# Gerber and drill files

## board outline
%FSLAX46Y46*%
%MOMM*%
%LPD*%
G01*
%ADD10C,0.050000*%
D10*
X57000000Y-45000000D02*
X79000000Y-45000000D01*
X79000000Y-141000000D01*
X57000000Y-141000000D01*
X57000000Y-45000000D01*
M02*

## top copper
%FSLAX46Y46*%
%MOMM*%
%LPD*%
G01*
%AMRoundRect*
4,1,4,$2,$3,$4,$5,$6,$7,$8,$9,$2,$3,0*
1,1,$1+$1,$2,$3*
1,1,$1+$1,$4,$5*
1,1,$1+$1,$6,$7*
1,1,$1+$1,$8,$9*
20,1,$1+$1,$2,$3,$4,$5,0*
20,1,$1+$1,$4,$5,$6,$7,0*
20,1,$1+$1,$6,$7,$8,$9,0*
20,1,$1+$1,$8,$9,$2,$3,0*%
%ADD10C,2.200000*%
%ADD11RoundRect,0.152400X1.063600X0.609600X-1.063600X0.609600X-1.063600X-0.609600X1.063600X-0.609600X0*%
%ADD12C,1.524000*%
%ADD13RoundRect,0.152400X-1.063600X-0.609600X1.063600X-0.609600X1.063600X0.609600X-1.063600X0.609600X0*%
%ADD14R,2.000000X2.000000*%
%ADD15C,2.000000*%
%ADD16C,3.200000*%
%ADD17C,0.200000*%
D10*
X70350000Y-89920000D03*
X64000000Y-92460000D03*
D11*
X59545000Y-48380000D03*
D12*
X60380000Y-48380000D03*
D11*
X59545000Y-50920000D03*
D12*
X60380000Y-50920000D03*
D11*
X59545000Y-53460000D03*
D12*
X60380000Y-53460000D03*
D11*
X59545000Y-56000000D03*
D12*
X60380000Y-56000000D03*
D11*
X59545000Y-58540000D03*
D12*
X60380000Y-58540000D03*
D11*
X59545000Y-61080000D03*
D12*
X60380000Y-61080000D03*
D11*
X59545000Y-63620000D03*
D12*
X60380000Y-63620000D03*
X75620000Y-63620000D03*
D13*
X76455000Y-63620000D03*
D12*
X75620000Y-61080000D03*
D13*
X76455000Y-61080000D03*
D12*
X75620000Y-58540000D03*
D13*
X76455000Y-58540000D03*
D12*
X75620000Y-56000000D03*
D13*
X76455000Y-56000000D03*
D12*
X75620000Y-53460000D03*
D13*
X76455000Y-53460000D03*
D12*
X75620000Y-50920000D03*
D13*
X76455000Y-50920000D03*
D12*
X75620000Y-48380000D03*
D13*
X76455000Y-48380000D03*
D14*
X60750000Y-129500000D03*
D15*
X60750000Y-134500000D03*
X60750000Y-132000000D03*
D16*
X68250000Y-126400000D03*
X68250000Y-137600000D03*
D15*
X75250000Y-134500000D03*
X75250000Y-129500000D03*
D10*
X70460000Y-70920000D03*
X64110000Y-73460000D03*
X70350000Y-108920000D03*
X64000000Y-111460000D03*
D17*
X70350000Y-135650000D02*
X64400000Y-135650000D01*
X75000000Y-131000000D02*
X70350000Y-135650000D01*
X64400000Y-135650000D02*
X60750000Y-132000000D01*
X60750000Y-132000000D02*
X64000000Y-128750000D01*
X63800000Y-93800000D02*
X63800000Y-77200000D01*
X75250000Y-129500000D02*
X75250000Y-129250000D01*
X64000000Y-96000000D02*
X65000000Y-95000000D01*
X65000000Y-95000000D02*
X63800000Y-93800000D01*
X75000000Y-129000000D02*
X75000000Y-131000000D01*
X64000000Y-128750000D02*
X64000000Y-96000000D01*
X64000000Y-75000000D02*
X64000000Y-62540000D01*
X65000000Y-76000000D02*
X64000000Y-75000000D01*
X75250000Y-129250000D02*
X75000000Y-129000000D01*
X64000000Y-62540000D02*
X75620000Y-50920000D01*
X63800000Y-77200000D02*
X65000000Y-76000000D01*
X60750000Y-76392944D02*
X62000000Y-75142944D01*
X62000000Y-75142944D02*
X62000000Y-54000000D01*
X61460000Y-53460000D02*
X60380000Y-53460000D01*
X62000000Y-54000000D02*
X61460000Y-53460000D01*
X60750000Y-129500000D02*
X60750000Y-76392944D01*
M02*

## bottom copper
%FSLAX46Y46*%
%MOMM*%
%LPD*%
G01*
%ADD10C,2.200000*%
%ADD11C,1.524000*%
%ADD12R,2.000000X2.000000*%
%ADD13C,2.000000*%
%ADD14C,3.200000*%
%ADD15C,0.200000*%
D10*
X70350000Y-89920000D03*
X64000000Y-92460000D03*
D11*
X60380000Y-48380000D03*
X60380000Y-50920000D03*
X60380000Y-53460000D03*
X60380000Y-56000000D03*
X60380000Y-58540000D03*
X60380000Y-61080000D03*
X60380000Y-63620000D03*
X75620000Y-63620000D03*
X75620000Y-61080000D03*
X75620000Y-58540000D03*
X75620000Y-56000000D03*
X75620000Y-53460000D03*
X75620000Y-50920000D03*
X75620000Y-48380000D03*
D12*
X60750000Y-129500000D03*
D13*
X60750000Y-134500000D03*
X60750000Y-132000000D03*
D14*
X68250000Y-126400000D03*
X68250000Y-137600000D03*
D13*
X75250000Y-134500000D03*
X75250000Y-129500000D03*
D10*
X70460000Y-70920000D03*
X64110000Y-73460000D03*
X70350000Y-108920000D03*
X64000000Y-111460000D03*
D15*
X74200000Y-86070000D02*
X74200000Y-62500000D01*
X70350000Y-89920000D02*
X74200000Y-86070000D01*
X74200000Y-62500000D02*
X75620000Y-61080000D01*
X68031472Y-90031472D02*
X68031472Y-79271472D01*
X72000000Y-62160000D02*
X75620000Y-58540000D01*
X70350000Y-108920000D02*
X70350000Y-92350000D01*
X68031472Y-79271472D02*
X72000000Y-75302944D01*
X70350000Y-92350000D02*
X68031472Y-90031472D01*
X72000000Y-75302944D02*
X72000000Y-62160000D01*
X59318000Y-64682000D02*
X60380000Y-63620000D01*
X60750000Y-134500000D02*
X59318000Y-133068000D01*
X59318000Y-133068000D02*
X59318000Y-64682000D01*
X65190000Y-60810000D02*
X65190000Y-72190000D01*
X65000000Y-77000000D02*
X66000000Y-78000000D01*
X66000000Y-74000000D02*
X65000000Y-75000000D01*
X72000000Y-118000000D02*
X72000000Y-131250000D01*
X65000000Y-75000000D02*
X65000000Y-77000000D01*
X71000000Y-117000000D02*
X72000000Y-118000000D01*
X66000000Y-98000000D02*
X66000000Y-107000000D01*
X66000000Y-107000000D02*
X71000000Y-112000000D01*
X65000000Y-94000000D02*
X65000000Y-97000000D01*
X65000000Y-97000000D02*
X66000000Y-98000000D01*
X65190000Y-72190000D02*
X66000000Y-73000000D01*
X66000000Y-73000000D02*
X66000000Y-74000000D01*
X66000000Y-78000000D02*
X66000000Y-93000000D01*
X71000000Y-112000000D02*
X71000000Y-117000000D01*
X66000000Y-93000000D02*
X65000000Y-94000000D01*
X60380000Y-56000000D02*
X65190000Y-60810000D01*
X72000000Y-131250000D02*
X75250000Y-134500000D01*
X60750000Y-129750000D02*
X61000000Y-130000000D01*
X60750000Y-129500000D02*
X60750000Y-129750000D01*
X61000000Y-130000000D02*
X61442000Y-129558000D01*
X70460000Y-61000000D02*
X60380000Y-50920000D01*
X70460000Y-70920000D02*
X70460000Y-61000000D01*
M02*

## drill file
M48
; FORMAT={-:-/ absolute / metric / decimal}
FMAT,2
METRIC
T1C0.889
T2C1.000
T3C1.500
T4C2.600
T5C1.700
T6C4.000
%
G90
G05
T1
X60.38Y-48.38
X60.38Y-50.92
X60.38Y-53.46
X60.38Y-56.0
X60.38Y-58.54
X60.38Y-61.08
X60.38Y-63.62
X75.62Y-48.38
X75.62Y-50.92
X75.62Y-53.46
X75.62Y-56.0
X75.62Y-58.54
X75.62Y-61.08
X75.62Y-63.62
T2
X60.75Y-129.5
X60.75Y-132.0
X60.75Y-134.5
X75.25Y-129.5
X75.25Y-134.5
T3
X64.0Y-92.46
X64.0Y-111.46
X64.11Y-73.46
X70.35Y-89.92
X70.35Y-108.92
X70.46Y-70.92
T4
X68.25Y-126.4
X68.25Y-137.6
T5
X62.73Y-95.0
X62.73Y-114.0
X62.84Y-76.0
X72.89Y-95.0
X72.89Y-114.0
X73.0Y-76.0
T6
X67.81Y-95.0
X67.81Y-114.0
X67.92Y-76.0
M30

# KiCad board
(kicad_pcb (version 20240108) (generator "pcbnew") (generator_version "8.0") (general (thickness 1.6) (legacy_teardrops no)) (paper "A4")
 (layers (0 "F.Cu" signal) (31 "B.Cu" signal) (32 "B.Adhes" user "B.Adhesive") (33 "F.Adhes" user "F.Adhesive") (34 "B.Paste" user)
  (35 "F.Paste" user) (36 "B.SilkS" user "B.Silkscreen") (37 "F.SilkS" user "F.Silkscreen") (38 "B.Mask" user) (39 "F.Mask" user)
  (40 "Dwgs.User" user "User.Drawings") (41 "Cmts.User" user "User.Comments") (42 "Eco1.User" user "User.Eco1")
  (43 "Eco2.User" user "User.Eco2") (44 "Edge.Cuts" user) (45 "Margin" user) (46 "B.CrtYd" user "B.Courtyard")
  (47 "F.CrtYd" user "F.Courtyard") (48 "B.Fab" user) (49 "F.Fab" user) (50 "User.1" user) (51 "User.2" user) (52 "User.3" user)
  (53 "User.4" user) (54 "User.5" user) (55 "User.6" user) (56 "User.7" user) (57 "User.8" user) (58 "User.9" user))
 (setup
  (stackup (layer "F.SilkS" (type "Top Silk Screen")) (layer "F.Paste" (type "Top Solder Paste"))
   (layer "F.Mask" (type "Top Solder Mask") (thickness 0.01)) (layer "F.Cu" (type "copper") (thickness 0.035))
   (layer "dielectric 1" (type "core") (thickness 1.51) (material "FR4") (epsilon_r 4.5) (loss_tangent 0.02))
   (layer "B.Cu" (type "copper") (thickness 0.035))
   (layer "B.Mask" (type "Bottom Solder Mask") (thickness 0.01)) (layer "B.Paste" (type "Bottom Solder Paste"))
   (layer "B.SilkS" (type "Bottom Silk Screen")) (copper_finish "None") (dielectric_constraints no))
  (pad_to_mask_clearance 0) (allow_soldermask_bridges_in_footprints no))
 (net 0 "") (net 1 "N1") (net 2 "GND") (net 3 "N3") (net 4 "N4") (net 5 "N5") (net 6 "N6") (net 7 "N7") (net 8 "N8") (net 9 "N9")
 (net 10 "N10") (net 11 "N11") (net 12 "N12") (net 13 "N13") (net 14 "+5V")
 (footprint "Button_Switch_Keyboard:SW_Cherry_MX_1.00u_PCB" (layer "F.Cu") (at 70.35 89.92)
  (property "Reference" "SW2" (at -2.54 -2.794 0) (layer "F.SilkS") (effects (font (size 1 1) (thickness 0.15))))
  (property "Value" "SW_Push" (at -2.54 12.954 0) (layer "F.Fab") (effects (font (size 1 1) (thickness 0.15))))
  (pad "" np_thru_hole circle (at -7.62 5.08) (size 1.7 1.7) (drill 1.7) (layers "*.Cu" "*.Mask"))
  (pad "" np_thru_hole circle (at -2.54 5.08) (size 4 4) (drill 4) (layers "*.Cu" "*.Mask"))
  (pad "" np_thru_hole circle (at 2.54 5.08) (size 1.7 1.7) (drill 1.7) (layers "*.Cu" "*.Mask"))
  (pad "1" thru_hole circle (at 0 0) (size 2.2 2.2) (drill 1.5) (layers "*.Cu" "*.Mask") (remove_unused_layers no) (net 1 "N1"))
  (pad "2" thru_hole circle (at -6.35 2.54) (size 2.2 2.2) (drill 1.5) (layers "*.Cu" "*.Mask") (remove_unused_layers no) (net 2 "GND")))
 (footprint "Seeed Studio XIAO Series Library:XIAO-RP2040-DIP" (layer "F.Cu") (at 68 56)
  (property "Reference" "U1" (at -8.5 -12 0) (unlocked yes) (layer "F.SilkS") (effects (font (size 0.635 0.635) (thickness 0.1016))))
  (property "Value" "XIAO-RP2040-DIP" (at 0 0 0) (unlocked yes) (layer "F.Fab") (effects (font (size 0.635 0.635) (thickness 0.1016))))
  (pad "1" smd roundrect (at -8.455 -7.62 180) (size 2.432 1.524) (layers "F.Cu" "F.Mask") (roundrect_rratio 0.1) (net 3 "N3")
   (thermal_bridge_angle 45))
  (pad "1" thru_hole circle (at -7.62 -7.62 180) (size 1.524 1.524) (drill 0.889) (layers "*.Cu" "*.Mask") (remove_unused_layers no)
   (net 3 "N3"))
  (pad "2" smd roundrect (at -8.455 -5.08 180) (size 2.432 1.524) (layers "F.Cu" "F.Mask") (roundrect_rratio 0.1) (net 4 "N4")
   (thermal_bridge_angle 45))
  (pad "2" thru_hole circle (at -7.62 -5.08 180) (size 1.524 1.524) (drill 0.889) (layers "*.Cu" "*.Mask") (remove_unused_layers no)
   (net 4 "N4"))
  (pad "3" smd roundrect (at -8.455 -2.54 180) (size 2.432 1.524) (layers "F.Cu" "F.Mask") (roundrect_rratio 0.1) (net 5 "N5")
   (thermal_bridge_angle 45))
  (pad "3" thru_hole circle (at -7.62 -2.54 180) (size 1.524 1.524) (drill 0.889) (layers "*.Cu" "*.Mask") (remove_unused_layers no)
   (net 5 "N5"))
  (pad "4" smd roundrect (at -8.455 0 180) (size 2.432 1.524) (layers "F.Cu" "F.Mask") (roundrect_rratio 0.1) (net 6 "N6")
   (thermal_bridge_angle 45))
  (pad "4" thru_hole circle (at -7.62 0 180) (size 1.524 1.524) (drill 0.889) (layers "*.Cu" "*.Mask") (remove_unused_layers no)
   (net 6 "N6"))
  (pad "5" smd roundrect (at -8.455 2.54 180) (size 2.432 1.524) (layers "F.Cu" "F.Mask") (roundrect_rratio 0.1) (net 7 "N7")
   (thermal_bridge_angle 45))
  (pad "5" thru_hole circle (at -7.62 2.54 180) (size 1.524 1.524) (drill 0.889) (layers "*.Cu" "*.Mask") (remove_unused_layers no)
   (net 7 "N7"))
  (pad "6" smd roundrect (at -8.455 5.08 180) (size 2.432 1.524) (layers "F.Cu" "F.Mask") (roundrect_rratio 0.1) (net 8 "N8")
   (thermal_bridge_angle 45))
  (pad "6" thru_hole circle (at -7.62 5.08 180) (size 1.524 1.524) (drill 0.889) (layers "*.Cu" "*.Mask") (remove_unused_layers no)
   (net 8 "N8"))
  (pad "7" smd roundrect (at -8.455 7.62 180) (size 2.432 1.524) (layers "F.Cu" "F.Mask") (roundrect_rratio 0.1) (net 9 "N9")
   (thermal_bridge_angle 45))
  (pad "7" thru_hole circle (at -7.62 7.62 180) (size 1.524 1.524) (drill 0.889) (layers "*.Cu" "*.Mask") (remove_unused_layers no)
   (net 9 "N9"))
  (pad "8" thru_hole circle (at 7.62 7.62) (size 1.524 1.524) (drill 0.889) (layers "*.Cu" "*.Mask") (remove_unused_layers no)
   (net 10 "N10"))
  (pad "8" smd roundrect (at 8.455 7.62) (size 2.432 1.524) (layers "F.Cu" "F.Mask") (roundrect_rratio 0.1) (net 10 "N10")
   (thermal_bridge_angle 45))
  (pad "9" thru_hole circle (at 7.62 5.08) (size 1.524 1.524) (drill 0.889) (layers "*.Cu" "*.Mask") (remove_unused_layers no) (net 1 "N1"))
  (pad "9" smd roundrect (at 8.455 5.08) (size 2.432 1.524) (layers "F.Cu" "F.Mask") (roundrect_rratio 0.1) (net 1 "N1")
   (thermal_bridge_angle 45))
  (pad "10" thru_hole circle (at 7.62 2.54) (size 1.524 1.524) (drill 0.889) (layers "*.Cu" "*.Mask") (remove_unused_layers no)
   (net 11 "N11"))
  (pad "10" smd roundrect (at 8.455 2.54) (size 2.432 1.524) (layers "F.Cu" "F.Mask") (roundrect_rratio 0.1) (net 11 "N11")
   (thermal_bridge_angle 45))
  (pad "11" thru_hole circle (at 7.62 0) (size 1.524 1.524) (drill 0.889) (layers "*.Cu" "*.Mask") (remove_unused_layers no) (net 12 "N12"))
  (pad "11" smd roundrect (at 8.455 0) (size 2.432 1.524) (layers "F.Cu" "F.Mask") (roundrect_rratio 0.1) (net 12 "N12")
   (thermal_bridge_angle 45))
  (pad "12" thru_hole circle (at 7.62 -2.54) (size 1.524 1.524) (drill 0.889) (layers "*.Cu" "*.Mask") (remove_unused_layers no)
   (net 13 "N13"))
  (pad "12" smd roundrect (at 8.455 -2.54) (size 2.432 1.524) (layers "F.Cu" "F.Mask") (roundrect_rratio 0.1) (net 13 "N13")
   (thermal_bridge_angle 45))
  (pad "13" thru_hole circle (at 7.62 -5.08) (size 1.524 1.524) (drill 0.889) (layers "*.Cu" "*.Mask") (remove_unused_layers no)
   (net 2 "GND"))
  (pad "13" smd roundrect (at 8.455 -5.08) (size 2.432 1.524) (layers "F.Cu" "F.Mask") (roundrect_rratio 0.1) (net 2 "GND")
   (thermal_bridge_angle 45))
  (pad "14" thru_hole circle (at 7.62 -7.62) (size 1.524 1.524) (drill 0.889) (layers "*.Cu" "*.Mask") (remove_unused_layers no)
   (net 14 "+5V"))
  (pad "14" smd roundrect (at 8.455 -7.62) (size 2.432 1.524) (layers "F.Cu" "F.Mask") (roundrect_rratio 0.1) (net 14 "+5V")
   (thermal_bridge_angle 45)))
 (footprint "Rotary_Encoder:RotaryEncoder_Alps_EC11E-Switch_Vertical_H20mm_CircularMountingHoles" (layer "F.Cu") (at 60.75 129.5)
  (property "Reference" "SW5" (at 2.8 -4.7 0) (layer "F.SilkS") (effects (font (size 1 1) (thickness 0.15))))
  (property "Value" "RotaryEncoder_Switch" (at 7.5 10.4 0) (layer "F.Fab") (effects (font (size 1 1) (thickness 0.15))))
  (pad "A" thru_hole rect (at 0 0) (size 2 2) (drill 1) (layers "*.Cu" "*.Mask") (remove_unused_layers no) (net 5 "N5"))
  (pad "B" thru_hole circle (at 0 5) (size 2 2) (drill 1) (layers "*.Cu" "*.Mask") (remove_unused_layers no) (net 9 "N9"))
  (pad "C" thru_hole circle (at 0 2.5) (size 2 2) (drill 1) (layers "*.Cu" "*.Mask") (remove_unused_layers no) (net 2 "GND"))
  (pad "MP" thru_hole circle (at 7.5 -3.1) (size 3.2 3.2) (drill 2.6) (layers "*.Cu" "*.Mask") (remove_unused_layers no))
  (pad "MP" thru_hole circle (at 7.5 8.1) (size 3.2 3.2) (drill 2.6) (layers "*.Cu" "*.Mask") (remove_unused_layers no))
  (pad "S1" thru_hole circle (at 14.5 5) (size 2 2) (drill 1) (layers "*.Cu" "*.Mask") (remove_unused_layers no) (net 6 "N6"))
  (pad "S2" thru_hole circle (at 14.5 0) (size 2 2) (drill 1) (layers "*.Cu" "*.Mask") (remove_unused_layers no) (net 2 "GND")))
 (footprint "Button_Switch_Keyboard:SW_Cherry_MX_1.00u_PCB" (layer "F.Cu") (at 70.46 70.92)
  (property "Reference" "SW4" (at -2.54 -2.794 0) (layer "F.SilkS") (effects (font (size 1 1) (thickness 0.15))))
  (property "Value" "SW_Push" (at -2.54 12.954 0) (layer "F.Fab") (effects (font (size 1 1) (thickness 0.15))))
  (pad "" np_thru_hole circle (at -7.62 5.08) (size 1.7 1.7) (drill 1.7) (layers "*.Cu" "*.Mask"))
  (pad "" np_thru_hole circle (at -2.54 5.08) (size 4 4) (drill 4) (layers "*.Cu" "*.Mask"))
  (pad "" np_thru_hole circle (at 2.54 5.08) (size 1.7 1.7) (drill 1.7) (layers "*.Cu" "*.Mask"))
  (pad "1" thru_hole circle (at 0 0) (size 2.2 2.2) (drill 1.5) (layers "*.Cu" "*.Mask") (remove_unused_layers no) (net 4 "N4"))
  (pad "2" thru_hole circle (at -6.35 2.54) (size 2.2 2.2) (drill 1.5) (layers "*.Cu" "*.Mask") (remove_unused_layers no) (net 2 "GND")))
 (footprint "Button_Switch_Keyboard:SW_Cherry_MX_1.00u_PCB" (layer "F.Cu") (at 70.35 108.92)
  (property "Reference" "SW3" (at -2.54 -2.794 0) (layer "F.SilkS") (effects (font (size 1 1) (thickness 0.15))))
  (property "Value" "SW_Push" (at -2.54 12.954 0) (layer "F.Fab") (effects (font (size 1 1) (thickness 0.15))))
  (pad "" np_thru_hole circle (at -7.62 5.08) (size 1.7 1.7) (drill 1.7) (layers "*.Cu" "*.Mask"))
  (pad "" np_thru_hole circle (at -2.54 5.08) (size 4 4) (drill 4) (layers "*.Cu" "*.Mask"))
  (pad "" np_thru_hole circle (at 2.54 5.08) (size 1.7 1.7) (drill 1.7) (layers "*.Cu" "*.Mask"))
  (pad "1" thru_hole circle (at 0 0) (size 2.2 2.2) (drill 1.5) (layers "*.Cu" "*.Mask") (remove_unused_layers no) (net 11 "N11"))
  (pad "2" thru_hole circle (at -6.35 2.54) (size 2.2 2.2) (drill 1.5) (layers "*.Cu" "*.Mask") (remove_unused_layers no) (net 2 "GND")))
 (gr_rect (start 57 45) (end 79 141) (stroke (width 0.05) (type default)) (fill none) (layer "Edge.Cuts"))
 (segment (start 74.2 86.07) (end 74.2 62.5) (width 0.2) (layer "B.Cu") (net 1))
 (segment (start 70.35 89.92) (end 74.2 86.07) (width 0.2) (layer "B.Cu") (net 1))
 (segment (start 74.2 62.5) (end 75.62 61.08) (width 0.2) (layer "B.Cu") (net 1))
 (segment (start 70.35 135.65) (end 64.4 135.65) (width 0.2) (layer "F.Cu") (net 2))
 (segment (start 75 131) (end 70.35 135.65) (width 0.2) (layer "F.Cu") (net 2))
 (segment (start 64.4 135.65) (end 60.75 132) (width 0.2) (layer "F.Cu") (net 2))
 (segment (start 60.75 132) (end 64 128.75) (width 0.2) (layer "F.Cu") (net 2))
 (segment (start 63.8 93.8) (end 63.8 77.2) (width 0.2) (layer "F.Cu") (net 2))
 (segment (start 75.25 129.5) (end 75.25 129.25) (width 0.2) (layer "F.Cu") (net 2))
 (segment (start 64 96) (end 65 95) (width 0.2) (layer "F.Cu") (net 2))
 (segment (start 65 95) (end 63.8 93.8) (width 0.2) (layer "F.Cu") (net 2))
 (segment (start 75 129) (end 75 131) (width 0.2) (layer "F.Cu") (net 2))
 (segment (start 64 128.75) (end 64 96) (width 0.2) (layer "F.Cu") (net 2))
 (segment (start 64 75) (end 64 62.54) (width 0.2) (layer "F.Cu") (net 2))
 (segment (start 65 76) (end 64 75) (width 0.2) (layer "F.Cu") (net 2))
 (segment (start 75.25 129.25) (end 75 129) (width 0.2) (layer "F.Cu") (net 2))
 (segment (start 64 62.54) (end 75.62 50.92) (width 0.2) (layer "F.Cu") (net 2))
 (segment (start 63.8 77.2) (end 65 76) (width 0.2) (layer "F.Cu") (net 2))
 (segment (start 68.031472 90.031472) (end 68.031472 79.271472) (width 0.2) (layer "B.Cu") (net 11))
 (segment (start 72 62.16) (end 75.62 58.54) (width 0.2) (layer "B.Cu") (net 11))
 (segment (start 70.35 108.92) (end 70.35 92.35) (width 0.2) (layer "B.Cu") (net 11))
 (segment (start 68.031472 79.271472) (end 72 75.302944) (width 0.2) (layer "B.Cu") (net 11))
 (segment (start 70.35 92.35) (end 68.031472 90.031472) (width 0.2) (layer "B.Cu") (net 11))
 (segment (start 72 75.302944) (end 72 62.16) (width 0.2) (layer "B.Cu") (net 11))
 (segment (start 59.318 64.682) (end 60.38 63.62) (width 0.2) (layer "B.Cu") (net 9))
 (segment (start 60.75 134.5) (end 59.318 133.068) (width 0.2) (layer "B.Cu") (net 9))
 (segment (start 59.318 133.068) (end 59.318 64.682) (width 0.2) (layer "B.Cu") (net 9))
 (segment (start 65.19 60.81) (end 65.19 72.19) (width 0.2) (layer "B.Cu") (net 6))
 (segment (start 65 77) (end 66 78) (width 0.2) (layer "B.Cu") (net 6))
 (segment (start 66 74) (end 65 75) (width 0.2) (layer "B.Cu") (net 6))
 (segment (start 72 118) (end 72 131.25) (width 0.2) (layer "B.Cu") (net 6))
 (segment (start 65 75) (end 65 77) (width 0.2) (layer "B.Cu") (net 6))
 (segment (start 71 117) (end 72 118) (width 0.2) (layer "B.Cu") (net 6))
 (segment (start 66 98) (end 66 107) (width 0.2) (layer "B.Cu") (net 6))
 (segment (start 66 107) (end 71 112) (width 0.2) (layer "B.Cu") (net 6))
 (segment (start 65 94) (end 65 97) (width 0.2) (layer "B.Cu") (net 6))
 (segment (start 65 97) (end 66 98) (width 0.2) (layer "B.Cu") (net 6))
 (segment (start 65.19 72.19) (end 66 73) (width 0.2) (layer "B.Cu") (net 6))
 (segment (start 66 73) (end 66 74) (width 0.2) (layer "B.Cu") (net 6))
 (segment (start 66 78) (end 66 93) (width 0.2) (layer "B.Cu") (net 6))
 (segment (start 71 112) (end 71 117) (width 0.2) (layer "B.Cu") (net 6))
 (segment (start 66 93) (end 65 94) (width 0.2) (layer "B.Cu") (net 6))
 (segment (start 60.38 56) (end 65.19 60.81) (width 0.2) (layer "B.Cu") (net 6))
 (segment (start 72 131.25) (end 75.25 134.5) (width 0.2) (layer "B.Cu") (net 6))
 (segment (start 60.75 76.392944) (end 62 75.142944) (width 0.2) (layer "F.Cu") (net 5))
 (segment (start 62 75.142944) (end 62 54) (width 0.2) (layer "F.Cu") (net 5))
 (segment (start 61.46 53.46) (end 60.38 53.46) (width 0.2) (layer "F.Cu") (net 5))
 (segment (start 62 54) (end 61.46 53.46) (width 0.2) (layer "F.Cu") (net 5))
 (segment (start 60.75 129.5) (end 60.75 76.392944) (width 0.2) (layer "F.Cu") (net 5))
 (segment (start 60.75 129.75) (end 61 130) (width 0.2) (layer "B.Cu") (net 5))
 (segment (start 60.75 129.5) (end 60.75 129.75) (width 0.2) (layer "B.Cu") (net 5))
 (segment (start 61 130) (end 61.442 129.558) (width 0.2) (layer "B.Cu") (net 5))
 (segment (start 70.46 61) (end 60.38 50.92) (width 0.2) (layer "B.Cu") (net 4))
 (segment (start 70.46 70.92) (end 70.46 61) (width 0.2) (layer "B.Cu") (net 4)))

